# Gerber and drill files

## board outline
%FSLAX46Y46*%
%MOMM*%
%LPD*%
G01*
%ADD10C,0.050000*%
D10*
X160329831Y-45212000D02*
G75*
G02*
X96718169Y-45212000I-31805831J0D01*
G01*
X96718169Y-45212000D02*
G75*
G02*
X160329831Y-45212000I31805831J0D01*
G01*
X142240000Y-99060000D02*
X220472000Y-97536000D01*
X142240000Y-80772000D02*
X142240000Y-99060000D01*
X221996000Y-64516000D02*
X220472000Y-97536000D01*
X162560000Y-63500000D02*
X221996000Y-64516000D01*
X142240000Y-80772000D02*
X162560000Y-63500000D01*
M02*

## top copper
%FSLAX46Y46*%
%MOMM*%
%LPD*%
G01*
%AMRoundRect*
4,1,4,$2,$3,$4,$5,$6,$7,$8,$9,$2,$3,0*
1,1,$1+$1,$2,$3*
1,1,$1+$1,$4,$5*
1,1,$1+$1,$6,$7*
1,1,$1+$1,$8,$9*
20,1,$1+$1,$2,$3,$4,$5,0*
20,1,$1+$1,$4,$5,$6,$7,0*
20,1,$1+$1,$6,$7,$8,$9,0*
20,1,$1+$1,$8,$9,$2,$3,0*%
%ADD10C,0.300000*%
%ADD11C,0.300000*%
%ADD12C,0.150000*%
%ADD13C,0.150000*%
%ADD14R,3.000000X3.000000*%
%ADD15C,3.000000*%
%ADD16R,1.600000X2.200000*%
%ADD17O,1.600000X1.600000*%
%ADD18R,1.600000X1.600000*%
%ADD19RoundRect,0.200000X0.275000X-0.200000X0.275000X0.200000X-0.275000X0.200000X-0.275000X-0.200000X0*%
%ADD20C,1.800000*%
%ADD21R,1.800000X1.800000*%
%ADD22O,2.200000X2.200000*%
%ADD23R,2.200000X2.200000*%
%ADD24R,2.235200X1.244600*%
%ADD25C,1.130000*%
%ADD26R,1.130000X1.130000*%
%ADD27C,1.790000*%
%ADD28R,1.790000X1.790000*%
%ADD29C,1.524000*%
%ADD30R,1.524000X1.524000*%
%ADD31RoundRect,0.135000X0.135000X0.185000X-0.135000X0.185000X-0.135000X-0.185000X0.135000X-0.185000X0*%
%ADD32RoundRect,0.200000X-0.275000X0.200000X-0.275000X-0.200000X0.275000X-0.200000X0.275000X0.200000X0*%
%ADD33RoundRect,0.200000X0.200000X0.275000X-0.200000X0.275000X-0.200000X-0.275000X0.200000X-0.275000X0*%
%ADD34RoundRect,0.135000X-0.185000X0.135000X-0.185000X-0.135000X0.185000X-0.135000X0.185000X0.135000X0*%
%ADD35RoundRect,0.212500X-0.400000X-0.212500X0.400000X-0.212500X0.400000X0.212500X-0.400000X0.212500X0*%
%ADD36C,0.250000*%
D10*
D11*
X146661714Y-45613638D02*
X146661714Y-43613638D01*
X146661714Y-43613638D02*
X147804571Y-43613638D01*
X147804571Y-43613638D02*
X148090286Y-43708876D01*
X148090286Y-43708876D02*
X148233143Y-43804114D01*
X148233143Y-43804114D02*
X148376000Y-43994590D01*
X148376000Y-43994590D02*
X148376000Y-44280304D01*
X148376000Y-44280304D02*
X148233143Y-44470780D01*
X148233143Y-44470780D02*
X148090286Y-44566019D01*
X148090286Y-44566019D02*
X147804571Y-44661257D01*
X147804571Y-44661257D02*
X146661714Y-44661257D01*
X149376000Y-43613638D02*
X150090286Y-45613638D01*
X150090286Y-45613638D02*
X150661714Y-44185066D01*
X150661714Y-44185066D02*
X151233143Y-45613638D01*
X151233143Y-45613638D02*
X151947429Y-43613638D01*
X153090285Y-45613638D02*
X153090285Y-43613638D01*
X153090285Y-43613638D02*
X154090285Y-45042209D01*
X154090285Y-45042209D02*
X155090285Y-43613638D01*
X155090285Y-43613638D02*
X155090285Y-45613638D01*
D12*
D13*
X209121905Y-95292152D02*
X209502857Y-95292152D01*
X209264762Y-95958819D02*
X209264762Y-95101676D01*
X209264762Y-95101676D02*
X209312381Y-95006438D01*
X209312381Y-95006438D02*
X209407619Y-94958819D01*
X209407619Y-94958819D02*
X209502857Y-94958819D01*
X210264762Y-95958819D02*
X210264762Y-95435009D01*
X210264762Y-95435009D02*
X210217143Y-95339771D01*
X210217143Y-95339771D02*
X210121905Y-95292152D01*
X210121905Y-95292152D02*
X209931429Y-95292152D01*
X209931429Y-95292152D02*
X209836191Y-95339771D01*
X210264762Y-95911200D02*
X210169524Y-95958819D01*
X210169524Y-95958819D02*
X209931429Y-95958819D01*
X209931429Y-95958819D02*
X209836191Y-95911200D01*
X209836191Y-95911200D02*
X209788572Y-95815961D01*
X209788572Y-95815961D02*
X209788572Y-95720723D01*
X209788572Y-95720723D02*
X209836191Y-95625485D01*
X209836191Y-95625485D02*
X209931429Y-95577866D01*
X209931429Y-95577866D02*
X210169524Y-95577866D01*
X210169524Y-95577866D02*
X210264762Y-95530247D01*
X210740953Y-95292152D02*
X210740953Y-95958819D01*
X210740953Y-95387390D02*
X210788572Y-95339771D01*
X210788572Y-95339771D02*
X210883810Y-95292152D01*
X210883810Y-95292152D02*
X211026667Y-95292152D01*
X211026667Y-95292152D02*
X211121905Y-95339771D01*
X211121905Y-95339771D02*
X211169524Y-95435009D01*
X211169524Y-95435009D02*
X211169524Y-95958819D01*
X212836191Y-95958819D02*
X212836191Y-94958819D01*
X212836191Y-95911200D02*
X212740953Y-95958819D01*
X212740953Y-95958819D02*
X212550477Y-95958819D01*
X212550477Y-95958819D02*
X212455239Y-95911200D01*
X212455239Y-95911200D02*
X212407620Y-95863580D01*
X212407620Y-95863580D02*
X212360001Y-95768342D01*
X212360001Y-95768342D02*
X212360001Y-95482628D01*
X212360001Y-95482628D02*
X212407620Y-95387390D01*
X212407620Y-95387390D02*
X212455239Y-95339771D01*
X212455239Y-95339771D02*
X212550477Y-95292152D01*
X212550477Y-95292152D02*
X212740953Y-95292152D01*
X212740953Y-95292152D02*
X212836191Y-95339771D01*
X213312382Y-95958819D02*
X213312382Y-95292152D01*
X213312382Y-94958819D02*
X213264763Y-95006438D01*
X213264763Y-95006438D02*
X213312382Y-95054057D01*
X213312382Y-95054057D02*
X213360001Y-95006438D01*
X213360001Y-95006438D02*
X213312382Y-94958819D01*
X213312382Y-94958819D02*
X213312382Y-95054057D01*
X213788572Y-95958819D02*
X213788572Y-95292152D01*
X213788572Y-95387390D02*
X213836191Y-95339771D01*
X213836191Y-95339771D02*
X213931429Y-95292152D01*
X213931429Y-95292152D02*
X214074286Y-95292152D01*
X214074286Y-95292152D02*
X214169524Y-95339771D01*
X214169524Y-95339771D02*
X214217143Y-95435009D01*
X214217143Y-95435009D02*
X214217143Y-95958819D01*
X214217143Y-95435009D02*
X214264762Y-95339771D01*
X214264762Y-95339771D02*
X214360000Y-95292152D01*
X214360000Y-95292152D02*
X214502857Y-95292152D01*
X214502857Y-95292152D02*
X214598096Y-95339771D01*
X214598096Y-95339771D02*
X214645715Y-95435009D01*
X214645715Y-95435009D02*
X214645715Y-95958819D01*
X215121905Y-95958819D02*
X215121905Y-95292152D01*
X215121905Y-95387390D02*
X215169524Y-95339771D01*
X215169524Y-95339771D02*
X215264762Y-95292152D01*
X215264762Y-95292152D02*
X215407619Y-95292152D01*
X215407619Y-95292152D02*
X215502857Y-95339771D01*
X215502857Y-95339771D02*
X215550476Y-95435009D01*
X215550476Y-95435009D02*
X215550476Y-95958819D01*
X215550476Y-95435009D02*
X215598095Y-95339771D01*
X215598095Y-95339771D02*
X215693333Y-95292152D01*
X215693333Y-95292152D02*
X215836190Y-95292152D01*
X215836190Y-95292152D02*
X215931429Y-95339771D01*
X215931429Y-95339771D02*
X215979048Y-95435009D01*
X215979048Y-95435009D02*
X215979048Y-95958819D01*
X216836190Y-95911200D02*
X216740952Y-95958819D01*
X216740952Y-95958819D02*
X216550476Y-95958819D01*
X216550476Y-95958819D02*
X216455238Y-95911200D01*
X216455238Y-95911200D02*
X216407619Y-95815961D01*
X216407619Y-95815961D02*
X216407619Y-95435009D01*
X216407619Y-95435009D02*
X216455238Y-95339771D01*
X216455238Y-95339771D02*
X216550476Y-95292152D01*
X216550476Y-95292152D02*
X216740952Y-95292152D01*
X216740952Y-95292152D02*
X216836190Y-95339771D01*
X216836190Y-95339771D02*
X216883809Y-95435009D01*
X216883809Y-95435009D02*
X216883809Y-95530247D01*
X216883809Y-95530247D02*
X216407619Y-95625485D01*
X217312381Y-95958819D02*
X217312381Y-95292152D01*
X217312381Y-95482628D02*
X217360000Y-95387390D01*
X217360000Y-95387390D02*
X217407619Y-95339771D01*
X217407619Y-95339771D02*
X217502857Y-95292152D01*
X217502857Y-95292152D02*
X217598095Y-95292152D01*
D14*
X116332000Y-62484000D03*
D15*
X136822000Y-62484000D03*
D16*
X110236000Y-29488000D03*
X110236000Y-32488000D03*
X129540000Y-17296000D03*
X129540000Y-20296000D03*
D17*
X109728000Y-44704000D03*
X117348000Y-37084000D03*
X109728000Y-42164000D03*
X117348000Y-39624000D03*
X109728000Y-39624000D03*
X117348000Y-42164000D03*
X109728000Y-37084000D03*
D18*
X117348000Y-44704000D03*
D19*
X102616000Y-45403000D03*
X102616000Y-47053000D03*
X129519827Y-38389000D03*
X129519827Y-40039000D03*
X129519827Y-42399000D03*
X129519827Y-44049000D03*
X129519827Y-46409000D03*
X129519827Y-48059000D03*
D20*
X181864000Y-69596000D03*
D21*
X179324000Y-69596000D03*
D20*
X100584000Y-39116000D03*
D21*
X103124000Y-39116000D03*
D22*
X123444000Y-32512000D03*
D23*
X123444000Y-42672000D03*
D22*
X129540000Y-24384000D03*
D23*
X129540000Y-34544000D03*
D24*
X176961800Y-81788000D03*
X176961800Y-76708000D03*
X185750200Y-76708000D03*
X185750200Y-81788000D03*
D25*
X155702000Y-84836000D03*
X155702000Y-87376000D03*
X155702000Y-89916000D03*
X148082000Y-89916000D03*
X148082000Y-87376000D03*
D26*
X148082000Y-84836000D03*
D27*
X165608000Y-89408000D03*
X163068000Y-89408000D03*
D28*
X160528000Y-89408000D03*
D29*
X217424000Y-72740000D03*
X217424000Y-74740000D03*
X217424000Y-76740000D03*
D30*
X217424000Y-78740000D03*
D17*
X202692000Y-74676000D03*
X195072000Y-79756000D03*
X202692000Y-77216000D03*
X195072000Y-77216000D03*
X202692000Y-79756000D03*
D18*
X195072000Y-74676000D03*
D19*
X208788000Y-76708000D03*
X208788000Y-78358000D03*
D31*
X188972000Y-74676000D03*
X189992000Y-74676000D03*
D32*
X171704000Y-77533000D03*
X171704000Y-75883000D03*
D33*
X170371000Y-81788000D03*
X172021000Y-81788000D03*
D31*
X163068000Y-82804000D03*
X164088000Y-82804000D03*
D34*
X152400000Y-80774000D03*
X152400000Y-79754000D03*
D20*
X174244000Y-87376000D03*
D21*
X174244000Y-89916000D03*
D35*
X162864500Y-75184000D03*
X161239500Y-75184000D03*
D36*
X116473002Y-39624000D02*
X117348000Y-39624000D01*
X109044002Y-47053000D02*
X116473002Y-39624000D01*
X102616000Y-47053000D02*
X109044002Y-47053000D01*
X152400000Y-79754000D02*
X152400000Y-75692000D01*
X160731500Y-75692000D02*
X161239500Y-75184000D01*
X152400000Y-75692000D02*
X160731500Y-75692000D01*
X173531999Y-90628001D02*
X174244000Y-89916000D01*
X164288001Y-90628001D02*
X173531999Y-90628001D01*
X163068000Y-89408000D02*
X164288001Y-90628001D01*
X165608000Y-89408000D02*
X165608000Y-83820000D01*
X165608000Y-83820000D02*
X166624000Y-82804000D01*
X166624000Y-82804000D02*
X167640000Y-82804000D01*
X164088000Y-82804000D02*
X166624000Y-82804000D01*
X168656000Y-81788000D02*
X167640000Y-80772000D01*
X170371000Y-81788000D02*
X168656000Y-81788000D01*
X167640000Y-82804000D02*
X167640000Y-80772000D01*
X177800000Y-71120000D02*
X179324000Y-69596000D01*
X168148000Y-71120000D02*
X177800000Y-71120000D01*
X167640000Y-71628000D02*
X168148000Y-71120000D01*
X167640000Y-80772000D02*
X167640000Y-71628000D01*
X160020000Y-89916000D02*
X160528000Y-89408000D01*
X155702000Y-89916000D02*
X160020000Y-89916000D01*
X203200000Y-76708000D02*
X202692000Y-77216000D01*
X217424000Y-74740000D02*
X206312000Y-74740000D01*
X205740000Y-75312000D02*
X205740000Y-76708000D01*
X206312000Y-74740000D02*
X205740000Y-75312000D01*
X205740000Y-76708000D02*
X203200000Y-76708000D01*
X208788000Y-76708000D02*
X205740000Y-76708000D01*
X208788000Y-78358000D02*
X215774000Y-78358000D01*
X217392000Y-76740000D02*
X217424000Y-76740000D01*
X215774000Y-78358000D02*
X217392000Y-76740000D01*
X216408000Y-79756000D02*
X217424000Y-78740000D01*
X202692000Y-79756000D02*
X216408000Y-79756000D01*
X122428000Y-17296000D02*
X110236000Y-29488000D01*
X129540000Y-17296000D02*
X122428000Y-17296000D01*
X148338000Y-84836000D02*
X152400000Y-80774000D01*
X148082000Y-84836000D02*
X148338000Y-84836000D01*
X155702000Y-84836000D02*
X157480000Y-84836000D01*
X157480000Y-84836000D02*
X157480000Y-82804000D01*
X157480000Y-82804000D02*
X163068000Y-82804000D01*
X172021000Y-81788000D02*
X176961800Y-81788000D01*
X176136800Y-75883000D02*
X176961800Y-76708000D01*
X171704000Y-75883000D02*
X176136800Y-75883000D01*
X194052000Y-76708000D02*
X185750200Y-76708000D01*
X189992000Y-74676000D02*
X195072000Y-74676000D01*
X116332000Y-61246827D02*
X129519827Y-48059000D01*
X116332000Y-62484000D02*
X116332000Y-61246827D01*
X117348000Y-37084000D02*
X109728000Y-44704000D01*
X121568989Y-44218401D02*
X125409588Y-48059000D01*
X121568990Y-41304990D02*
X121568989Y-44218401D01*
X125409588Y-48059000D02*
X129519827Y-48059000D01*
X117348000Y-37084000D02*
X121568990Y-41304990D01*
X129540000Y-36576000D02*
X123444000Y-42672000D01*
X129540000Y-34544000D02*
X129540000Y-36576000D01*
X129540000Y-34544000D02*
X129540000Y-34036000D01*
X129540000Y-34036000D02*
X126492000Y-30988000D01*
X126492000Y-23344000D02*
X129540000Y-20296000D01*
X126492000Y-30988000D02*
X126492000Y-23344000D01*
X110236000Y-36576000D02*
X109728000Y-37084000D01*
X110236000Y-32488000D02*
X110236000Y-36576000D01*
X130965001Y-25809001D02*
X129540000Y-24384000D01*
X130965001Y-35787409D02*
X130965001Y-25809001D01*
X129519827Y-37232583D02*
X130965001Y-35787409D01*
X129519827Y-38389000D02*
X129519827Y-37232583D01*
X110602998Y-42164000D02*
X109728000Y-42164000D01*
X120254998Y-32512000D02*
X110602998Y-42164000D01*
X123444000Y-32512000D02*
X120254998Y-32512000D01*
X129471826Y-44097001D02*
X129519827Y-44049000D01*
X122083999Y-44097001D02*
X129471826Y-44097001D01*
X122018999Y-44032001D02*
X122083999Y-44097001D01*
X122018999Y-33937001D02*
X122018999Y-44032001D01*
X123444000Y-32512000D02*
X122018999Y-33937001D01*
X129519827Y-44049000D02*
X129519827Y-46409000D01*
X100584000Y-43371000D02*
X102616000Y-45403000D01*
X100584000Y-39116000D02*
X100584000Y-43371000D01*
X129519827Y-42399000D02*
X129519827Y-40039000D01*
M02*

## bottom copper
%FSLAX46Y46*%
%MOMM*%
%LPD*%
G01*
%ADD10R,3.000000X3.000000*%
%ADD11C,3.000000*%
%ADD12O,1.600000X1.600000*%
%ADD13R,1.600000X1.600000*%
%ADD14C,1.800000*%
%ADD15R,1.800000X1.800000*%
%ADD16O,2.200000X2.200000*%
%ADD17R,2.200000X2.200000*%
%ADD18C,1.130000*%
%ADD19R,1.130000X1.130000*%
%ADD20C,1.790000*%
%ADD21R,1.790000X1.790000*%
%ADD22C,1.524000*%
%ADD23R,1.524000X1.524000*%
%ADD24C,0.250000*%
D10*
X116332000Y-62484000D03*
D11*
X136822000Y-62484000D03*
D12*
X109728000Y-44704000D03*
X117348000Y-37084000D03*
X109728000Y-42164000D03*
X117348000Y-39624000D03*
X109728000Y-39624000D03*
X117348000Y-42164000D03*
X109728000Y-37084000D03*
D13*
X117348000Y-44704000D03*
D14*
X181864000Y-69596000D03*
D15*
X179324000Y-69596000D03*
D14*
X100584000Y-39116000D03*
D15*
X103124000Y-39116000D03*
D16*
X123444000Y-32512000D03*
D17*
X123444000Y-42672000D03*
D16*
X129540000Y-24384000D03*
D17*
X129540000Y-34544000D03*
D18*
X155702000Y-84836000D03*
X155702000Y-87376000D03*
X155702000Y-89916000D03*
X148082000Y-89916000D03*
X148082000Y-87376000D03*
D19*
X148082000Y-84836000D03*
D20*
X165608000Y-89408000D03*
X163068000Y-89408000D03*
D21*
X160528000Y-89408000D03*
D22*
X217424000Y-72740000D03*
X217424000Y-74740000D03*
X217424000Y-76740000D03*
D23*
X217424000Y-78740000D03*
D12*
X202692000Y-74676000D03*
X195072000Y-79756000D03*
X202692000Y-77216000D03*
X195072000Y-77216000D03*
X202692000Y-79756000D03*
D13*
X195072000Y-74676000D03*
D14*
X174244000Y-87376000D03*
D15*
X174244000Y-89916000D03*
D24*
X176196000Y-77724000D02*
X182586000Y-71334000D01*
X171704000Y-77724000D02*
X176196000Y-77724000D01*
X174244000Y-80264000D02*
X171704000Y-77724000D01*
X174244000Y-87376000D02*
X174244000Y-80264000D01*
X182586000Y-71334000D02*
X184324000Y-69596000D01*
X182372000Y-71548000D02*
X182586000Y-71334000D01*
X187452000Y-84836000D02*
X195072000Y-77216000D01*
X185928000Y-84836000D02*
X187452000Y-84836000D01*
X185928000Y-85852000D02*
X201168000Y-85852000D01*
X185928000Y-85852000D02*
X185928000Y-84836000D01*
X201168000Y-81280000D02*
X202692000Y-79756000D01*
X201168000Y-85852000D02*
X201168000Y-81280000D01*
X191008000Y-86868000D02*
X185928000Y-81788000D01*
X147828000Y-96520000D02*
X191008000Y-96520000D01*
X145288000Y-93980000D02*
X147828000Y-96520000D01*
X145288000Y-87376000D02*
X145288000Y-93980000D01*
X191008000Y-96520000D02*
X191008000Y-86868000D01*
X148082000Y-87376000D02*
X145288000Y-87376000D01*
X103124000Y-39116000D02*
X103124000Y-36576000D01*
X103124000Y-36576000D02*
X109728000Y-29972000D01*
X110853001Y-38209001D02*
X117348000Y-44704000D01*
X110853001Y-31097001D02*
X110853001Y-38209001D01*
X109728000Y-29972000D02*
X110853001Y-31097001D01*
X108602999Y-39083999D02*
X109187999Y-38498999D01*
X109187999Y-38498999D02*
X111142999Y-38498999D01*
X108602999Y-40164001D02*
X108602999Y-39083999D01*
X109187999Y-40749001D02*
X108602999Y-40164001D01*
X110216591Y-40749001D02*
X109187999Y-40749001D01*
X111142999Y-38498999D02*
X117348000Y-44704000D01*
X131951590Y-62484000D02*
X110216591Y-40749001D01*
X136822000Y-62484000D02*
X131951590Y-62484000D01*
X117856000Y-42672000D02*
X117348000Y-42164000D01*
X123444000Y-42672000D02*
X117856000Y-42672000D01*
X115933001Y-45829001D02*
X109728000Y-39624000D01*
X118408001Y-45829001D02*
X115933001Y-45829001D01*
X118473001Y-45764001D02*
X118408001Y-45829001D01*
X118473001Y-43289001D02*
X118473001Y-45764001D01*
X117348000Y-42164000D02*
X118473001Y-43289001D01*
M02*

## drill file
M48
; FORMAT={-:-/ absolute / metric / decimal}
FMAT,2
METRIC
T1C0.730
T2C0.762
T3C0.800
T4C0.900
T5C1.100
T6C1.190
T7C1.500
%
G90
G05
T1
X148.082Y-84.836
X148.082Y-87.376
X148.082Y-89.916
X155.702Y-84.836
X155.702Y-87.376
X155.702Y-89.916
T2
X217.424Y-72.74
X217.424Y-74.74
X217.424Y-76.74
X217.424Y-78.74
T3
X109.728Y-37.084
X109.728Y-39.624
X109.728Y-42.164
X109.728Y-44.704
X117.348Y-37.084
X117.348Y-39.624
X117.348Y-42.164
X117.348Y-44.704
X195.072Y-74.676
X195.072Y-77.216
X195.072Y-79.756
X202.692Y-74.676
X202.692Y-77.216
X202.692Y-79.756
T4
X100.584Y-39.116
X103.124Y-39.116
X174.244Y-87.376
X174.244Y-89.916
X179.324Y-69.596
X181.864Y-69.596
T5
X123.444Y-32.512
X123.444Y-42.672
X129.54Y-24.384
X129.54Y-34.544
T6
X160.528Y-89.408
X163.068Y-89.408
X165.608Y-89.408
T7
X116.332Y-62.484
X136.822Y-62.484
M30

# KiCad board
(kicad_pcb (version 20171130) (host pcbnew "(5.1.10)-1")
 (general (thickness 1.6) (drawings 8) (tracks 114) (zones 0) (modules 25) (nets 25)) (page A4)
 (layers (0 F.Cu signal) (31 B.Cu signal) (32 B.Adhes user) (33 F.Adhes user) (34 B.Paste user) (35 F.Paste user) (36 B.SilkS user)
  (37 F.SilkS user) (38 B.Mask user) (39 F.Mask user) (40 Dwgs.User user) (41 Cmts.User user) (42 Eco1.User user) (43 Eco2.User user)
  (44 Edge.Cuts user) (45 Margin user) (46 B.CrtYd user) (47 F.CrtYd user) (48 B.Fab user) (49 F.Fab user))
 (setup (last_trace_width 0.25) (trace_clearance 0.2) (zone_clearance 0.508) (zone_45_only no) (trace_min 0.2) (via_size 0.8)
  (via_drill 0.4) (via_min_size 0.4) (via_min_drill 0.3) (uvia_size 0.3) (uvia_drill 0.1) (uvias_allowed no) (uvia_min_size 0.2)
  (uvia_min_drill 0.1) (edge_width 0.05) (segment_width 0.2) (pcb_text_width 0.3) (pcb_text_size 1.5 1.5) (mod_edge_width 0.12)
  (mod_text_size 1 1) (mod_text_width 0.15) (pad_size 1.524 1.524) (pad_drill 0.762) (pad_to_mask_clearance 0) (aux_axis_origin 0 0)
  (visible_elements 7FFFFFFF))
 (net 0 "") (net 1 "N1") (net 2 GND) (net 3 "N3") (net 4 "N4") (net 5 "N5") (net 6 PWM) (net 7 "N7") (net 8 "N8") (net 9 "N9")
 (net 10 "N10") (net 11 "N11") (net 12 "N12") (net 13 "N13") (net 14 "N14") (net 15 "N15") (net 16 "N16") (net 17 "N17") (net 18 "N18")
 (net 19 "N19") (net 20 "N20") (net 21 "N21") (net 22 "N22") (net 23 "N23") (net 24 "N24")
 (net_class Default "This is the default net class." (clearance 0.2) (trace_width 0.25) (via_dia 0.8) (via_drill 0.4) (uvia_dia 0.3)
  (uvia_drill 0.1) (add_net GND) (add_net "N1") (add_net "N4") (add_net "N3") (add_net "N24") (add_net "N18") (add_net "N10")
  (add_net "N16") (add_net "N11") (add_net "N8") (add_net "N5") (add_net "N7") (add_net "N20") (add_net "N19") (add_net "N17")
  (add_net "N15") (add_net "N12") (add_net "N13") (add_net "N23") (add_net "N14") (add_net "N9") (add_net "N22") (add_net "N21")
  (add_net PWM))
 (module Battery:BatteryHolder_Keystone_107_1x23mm (layer F.Cu) (at 116.332 62.484)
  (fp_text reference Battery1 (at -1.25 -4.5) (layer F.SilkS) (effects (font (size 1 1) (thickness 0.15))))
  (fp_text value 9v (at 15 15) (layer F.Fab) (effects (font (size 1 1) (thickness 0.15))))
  (pad 1 thru_hole rect (at 0 0) (size 3 3) (drill 1.5) (layers *.Cu *.Mask) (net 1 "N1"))
  (pad 2 thru_hole circle (at 20.49 0) (size 3 3) (drill 1.5) (layers *.Cu *.Mask) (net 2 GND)))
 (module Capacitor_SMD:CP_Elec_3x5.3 (layer F.Cu) (at 110.236 30.988 90)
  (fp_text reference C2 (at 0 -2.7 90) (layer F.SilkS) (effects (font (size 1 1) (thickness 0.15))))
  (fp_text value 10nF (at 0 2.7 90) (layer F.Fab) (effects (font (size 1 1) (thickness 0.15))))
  (pad 2 smd rect (at 1.5 0 90) (size 2.2 1.6) (layers F.Cu F.Paste F.Mask) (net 2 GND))
  (pad 1 smd rect (at -1.5 0 90) (size 2.2 1.6) (layers F.Cu F.Paste F.Mask) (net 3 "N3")))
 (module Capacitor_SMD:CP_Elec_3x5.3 (layer F.Cu) (at 129.54 18.796 90)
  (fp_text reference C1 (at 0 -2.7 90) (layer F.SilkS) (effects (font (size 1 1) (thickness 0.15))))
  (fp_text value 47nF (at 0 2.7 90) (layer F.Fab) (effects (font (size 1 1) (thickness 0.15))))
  (pad 2 smd rect (at 1.5 0 90) (size 2.2 1.6) (layers F.Cu F.Paste F.Mask) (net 2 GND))
  (pad 1 smd rect (at -1.5 0 90) (size 2.2 1.6) (layers F.Cu F.Paste F.Mask) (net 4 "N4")))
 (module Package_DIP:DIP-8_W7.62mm (layer F.Cu) (at 117.348 44.704 180)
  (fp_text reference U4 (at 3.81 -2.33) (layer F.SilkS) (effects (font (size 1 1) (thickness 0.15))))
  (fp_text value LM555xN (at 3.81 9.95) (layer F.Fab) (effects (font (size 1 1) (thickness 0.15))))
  (pad 8 thru_hole oval (at 7.62 0 180) (size 1.6 1.6) (drill 0.8) (layers *.Cu *.Mask) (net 1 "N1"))
  (pad 4 thru_hole oval (at 0 7.62 180) (size 1.6 1.6) (drill 0.8) (layers *.Cu *.Mask) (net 1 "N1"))
  (pad 7 thru_hole oval (at 7.62 2.54 180) (size 1.6 1.6) (drill 0.8) (layers *.Cu *.Mask) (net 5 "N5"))
  (pad 3 thru_hole oval (at 0 5.08 180) (size 1.6 1.6) (drill 0.8) (layers *.Cu *.Mask) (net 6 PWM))
  (pad 6 thru_hole oval (at 7.62 5.08 180) (size 1.6 1.6) (drill 0.8) (layers *.Cu *.Mask) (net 4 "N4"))
  (pad 2 thru_hole oval (at 0 2.54 180) (size 1.6 1.6) (drill 0.8) (layers *.Cu *.Mask) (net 4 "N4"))
  (pad 5 thru_hole oval (at 7.62 7.62 180) (size 1.6 1.6) (drill 0.8) (layers *.Cu *.Mask) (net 3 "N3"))
  (pad 1 thru_hole rect (at 0 0 180) (size 1.6 1.6) (drill 0.8) (layers *.Cu *.Mask) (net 2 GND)))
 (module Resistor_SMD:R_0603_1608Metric (layer F.Cu) (at 102.616 46.228 90)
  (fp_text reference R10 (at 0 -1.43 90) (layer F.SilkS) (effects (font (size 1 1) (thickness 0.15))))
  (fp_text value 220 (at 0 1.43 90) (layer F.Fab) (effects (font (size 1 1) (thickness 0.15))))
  (pad 2 smd roundrect (at 0.825 0 90) (size 0.8 0.95) (layers F.Cu F.Paste F.Mask) (roundrect_rratio 0.25) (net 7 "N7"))
  (pad 1 smd roundrect (at -0.825 0 90) (size 0.8 0.95) (layers F.Cu F.Paste F.Mask) (roundrect_rratio 0.25) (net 6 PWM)))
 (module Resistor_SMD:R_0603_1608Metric (layer F.Cu) (at 129.519827 39.214 90)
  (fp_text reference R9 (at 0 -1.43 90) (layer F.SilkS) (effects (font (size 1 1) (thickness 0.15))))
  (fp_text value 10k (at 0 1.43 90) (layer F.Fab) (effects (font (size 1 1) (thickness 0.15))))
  (pad 2 smd roundrect (at 0.825 0 90) (size 0.8 0.95) (layers F.Cu F.Paste F.Mask) (roundrect_rratio 0.25) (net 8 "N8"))
  (pad 1 smd roundrect (at -0.825 0 90) (size 0.8 0.95) (layers F.Cu F.Paste F.Mask) (roundrect_rratio 0.25) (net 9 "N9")))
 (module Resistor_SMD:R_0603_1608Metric (layer F.Cu) (at 129.519827 43.224 90)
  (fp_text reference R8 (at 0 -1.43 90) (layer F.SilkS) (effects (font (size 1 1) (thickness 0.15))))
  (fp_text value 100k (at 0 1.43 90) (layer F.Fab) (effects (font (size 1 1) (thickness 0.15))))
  (pad 2 smd roundrect (at 0.825 0 90) (size 0.8 0.95) (layers F.Cu F.Paste F.Mask) (roundrect_rratio 0.25) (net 9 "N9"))
  (pad 1 smd roundrect (at -0.825 0 90) (size 0.8 0.95) (layers F.Cu F.Paste F.Mask) (roundrect_rratio 0.25) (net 5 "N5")))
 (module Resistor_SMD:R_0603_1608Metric (layer F.Cu) (at 129.519827 47.234 90)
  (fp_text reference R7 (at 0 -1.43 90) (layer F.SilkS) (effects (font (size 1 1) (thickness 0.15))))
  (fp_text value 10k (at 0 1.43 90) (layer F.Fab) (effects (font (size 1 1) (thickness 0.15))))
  (pad 2 smd roundrect (at 0.825 0 90) (size 0.8 0.95) (layers F.Cu F.Paste F.Mask) (roundrect_rratio 0.25) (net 5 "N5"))
  (pad 1 smd roundrect (at -0.825 0 90) (size 0.8 0.95) (layers F.Cu F.Paste F.Mask) (roundrect_rratio 0.25) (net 1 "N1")))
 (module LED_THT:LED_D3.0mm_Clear (layer F.Cu) (at 179.324 69.596)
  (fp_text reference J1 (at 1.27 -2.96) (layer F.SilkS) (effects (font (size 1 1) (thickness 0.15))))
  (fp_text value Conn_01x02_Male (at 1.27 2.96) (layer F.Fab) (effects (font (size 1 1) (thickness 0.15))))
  (pad 2 thru_hole circle (at 2.54 0) (size 1.8 1.8) (drill 0.9) (layers *.Cu *.Mask) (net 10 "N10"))
  (pad 1 thru_hole rect (at 0 0) (size 1.8 1.8) (drill 0.9) (layers *.Cu *.Mask) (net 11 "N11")))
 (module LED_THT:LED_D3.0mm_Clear (layer F.Cu) (at 103.124 39.116 180)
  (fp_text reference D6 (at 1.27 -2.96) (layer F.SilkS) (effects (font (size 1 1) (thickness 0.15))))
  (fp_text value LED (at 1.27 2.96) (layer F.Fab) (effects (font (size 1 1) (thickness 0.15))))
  (pad 2 thru_hole circle (at 2.54 0 180) (size 1.8 1.8) (drill 0.9) (layers *.Cu *.Mask) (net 7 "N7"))
  (pad 1 thru_hole rect (at 0 0 180) (size 1.8 1.8) (drill 0.9) (layers *.Cu *.Mask) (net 2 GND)))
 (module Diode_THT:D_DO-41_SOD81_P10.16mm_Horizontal (layer F.Cu) (at 123.444 42.672 90)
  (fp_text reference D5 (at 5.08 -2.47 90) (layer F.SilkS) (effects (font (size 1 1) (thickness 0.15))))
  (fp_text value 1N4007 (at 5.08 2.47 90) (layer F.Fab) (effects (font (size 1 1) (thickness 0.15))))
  (pad 2 thru_hole oval (at 10.16 0 90) (size 2.2 2.2) (drill 1.1) (layers *.Cu *.Mask) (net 5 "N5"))
  (pad 1 thru_hole rect (at 0 0 90) (size 2.2 2.2) (drill 1.1) (layers *.Cu *.Mask) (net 4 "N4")))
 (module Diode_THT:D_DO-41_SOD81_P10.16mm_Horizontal (layer F.Cu) (at 129.54 34.544 90)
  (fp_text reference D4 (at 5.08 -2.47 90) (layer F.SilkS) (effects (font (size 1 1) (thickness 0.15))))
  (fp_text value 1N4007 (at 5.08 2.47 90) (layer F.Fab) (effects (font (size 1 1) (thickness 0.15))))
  (pad 2 thru_hole oval (at 10.16 0 90) (size 2.2 2.2) (drill 1.1) (layers *.Cu *.Mask) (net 8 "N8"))
  (pad 1 thru_hole rect (at 0 0 90) (size 2.2 2.2) (drill 1.1) (layers *.Cu *.Mask) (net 4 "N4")))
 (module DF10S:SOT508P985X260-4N (layer F.Cu) (at 181.356 79.248 180)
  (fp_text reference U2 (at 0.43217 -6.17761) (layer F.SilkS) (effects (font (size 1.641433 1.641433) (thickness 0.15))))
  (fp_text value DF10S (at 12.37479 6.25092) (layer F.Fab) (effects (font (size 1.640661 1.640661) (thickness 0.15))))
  (pad 4 smd rect (at 4.3942 -2.54 180) (size 2.2352 1.2446) (layers F.Cu F.Paste F.Mask) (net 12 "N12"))
  (pad 3 smd rect (at 4.3942 2.54 180) (size 2.2352 1.2446) (layers F.Cu F.Paste F.Mask) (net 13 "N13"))
  (pad 2 smd rect (at -4.3942 2.54 180) (size 2.2352 1.2446) (layers F.Cu F.Paste F.Mask) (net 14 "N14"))
  (pad 1 smd rect (at -4.3942 -2.54 180) (size 2.2352 1.2446) (layers F.Cu F.Paste F.Mask) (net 2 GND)))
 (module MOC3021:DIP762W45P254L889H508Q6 (layer F.Cu) (at 151.892 87.376)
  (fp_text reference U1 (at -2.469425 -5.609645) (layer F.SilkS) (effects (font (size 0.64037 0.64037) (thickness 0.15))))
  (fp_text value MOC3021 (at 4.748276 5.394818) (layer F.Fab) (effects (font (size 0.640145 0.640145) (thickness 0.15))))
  (pad 6 thru_hole circle (at 3.81 -2.54) (size 1.13 1.13) (drill 0.73) (layers *.Cu *.Mask) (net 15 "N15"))
  (pad 5 thru_hole circle (at 3.81 0) (size 1.13 1.13) (drill 0.73) (layers *.Cu *.Mask))
  (pad 4 thru_hole circle (at 3.81 2.54) (size 1.13 1.13) (drill 0.73) (layers *.Cu *.Mask) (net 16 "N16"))
  (pad 3 thru_hole circle (at -3.81 2.54) (size 1.13 1.13) (drill 0.73) (layers *.Cu *.Mask))
  (pad 2 thru_hole circle (at -3.81 0) (size 1.13 1.13) (drill 0.73) (layers *.Cu *.Mask) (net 2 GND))
  (pad 1 thru_hole rect (at -3.81 -2.54) (size 1.13 1.13) (drill 0.73) (layers *.Cu *.Mask) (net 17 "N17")))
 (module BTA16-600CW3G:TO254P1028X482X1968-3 (layer F.Cu) (at 160.528 89.408)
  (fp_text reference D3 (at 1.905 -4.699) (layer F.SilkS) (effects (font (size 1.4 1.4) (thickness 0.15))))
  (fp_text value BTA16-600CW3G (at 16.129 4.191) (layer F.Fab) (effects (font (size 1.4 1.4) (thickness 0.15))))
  (pad 3 thru_hole circle (at 5.08 0) (size 1.79 1.79) (drill 1.19) (layers *.Cu *.Mask) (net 11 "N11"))
  (pad 2 thru_hole circle (at 2.54 0) (size 1.79 1.79) (drill 1.19) (layers *.Cu *.Mask) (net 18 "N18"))
  (pad 1 thru_hole rect (at 0 0) (size 1.79 1.79) (drill 1.19) (layers *.Cu *.Mask) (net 16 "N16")))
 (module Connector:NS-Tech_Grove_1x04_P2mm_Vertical (layer F.Cu) (at 217.424 78.74 180)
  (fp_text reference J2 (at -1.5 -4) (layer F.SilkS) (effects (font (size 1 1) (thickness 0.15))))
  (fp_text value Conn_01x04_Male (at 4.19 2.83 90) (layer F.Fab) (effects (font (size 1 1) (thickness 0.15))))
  (pad 4 thru_hole circle (at 0 6 180) (size 1.524 1.524) (drill 0.762) (layers *.Cu *.Mask) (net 6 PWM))
  (pad 3 thru_hole circle (at 0 4 180) (size 1.524 1.524) (drill 0.762) (layers *.Cu *.Mask) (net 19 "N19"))
  (pad 2 thru_hole circle (at 0 2 180) (size 1.524 1.524) (drill 0.762) (layers *.Cu *.Mask) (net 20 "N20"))
  (pad 1 thru_hole rect (at 0 0 180) (size 1.524 1.524) (drill 0.762) (layers *.Cu *.Mask) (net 2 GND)))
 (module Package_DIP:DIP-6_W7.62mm (layer F.Cu) (at 195.072 74.676)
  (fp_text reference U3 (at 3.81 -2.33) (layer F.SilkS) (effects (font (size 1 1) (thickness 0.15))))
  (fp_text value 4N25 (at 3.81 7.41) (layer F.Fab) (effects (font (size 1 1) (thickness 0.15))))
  (pad 6 thru_hole oval (at 7.62 0) (size 1.6 1.6) (drill 0.8) (layers *.Cu *.Mask) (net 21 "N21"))
  (pad 3 thru_hole oval (at 0 5.08) (size 1.6 1.6) (drill 0.8) (layers *.Cu *.Mask) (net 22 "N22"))
  (pad 5 thru_hole oval (at 7.62 2.54) (size 1.6 1.6) (drill 0.8) (layers *.Cu *.Mask) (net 19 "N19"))
  (pad 2 thru_hole oval (at 0 2.54) (size 1.6 1.6) (drill 0.8) (layers *.Cu *.Mask) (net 2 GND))
  (pad 4 thru_hole oval (at 7.62 5.08) (size 1.6 1.6) (drill 0.8) (layers *.Cu *.Mask) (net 2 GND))
  (pad 1 thru_hole rect (at 0 0) (size 1.6 1.6) (drill 0.8) (layers *.Cu *.Mask) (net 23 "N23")))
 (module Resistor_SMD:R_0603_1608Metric (layer F.Cu) (at 208.788 77.533 90)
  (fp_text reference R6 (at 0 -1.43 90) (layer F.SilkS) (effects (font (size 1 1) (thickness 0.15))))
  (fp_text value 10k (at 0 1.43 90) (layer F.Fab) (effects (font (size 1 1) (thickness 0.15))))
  (pad 2 smd roundrect (at 0.825 0 90) (size 0.8 0.95) (layers F.Cu F.Paste F.Mask) (roundrect_rratio 0.25) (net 19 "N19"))
  (pad 1 smd roundrect (at -0.825 0 90) (size 0.8 0.95) (layers F.Cu F.Paste F.Mask) (roundrect_rratio 0.25) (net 20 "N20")))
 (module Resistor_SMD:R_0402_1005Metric (layer F.Cu) (at 189.482 74.676 180)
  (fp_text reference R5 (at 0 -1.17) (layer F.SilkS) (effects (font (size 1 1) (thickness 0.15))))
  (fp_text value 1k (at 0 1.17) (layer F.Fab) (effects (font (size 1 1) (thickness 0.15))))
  (pad 2 smd roundrect (at 0.51 0 180) (size 0.54 0.64) (layers F.Cu F.Paste F.Mask) (roundrect_rratio 0.25) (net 14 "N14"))
  (pad 1 smd roundrect (at -0.51 0 180) (size 0.54 0.64) (layers F.Cu F.Paste F.Mask) (roundrect_rratio 0.25) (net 23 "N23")))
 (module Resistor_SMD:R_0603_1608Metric (layer F.Cu) (at 171.704 76.708 270)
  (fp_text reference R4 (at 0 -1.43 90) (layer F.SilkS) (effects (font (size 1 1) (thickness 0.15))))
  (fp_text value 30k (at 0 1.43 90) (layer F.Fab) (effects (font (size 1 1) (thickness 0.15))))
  (pad 2 smd roundrect (at 0.825 0 270) (size 0.8 0.95) (layers F.Cu F.Paste F.Mask) (roundrect_rratio 0.25) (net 10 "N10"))
  (pad 1 smd roundrect (at -0.825 0 270) (size 0.8 0.95) (layers F.Cu F.Paste F.Mask) (roundrect_rratio 0.25) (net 13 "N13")))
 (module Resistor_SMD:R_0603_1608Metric (layer F.Cu) (at 171.196 81.788 180)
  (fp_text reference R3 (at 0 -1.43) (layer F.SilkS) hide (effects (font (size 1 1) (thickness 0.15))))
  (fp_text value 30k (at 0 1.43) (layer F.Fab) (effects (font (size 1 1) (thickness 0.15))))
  (pad 2 smd roundrect (at 0.825 0 180) (size 0.8 0.95) (layers F.Cu F.Paste F.Mask) (roundrect_rratio 0.25) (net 11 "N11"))
  (pad 1 smd roundrect (at -0.825 0 180) (size 0.8 0.95) (layers F.Cu F.Paste F.Mask) (roundrect_rratio 0.25) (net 12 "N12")))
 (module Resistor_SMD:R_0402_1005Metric (layer F.Cu) (at 163.578 82.804 180)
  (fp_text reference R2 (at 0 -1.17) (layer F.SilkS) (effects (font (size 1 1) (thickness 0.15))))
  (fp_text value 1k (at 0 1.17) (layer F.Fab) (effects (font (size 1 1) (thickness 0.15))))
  (pad 2 smd roundrect (at 0.51 0 180) (size 0.54 0.64) (layers F.Cu F.Paste F.Mask) (roundrect_rratio 0.25) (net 15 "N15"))
  (pad 1 smd roundrect (at -0.51 0 180) (size 0.54 0.64) (layers F.Cu F.Paste F.Mask) (roundrect_rratio 0.25) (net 11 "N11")))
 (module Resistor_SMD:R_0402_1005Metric (layer F.Cu) (at 152.4 80.264 270)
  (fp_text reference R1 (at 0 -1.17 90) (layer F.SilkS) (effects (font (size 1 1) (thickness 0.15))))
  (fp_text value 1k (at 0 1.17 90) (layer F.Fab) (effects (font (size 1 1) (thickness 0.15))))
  (pad 2 smd roundrect (at 0.51 0 270) (size 0.54 0.64) (layers F.Cu F.Paste F.Mask) (roundrect_rratio 0.25) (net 17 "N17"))
  (pad 1 smd roundrect (at -0.51 0 270) (size 0.54 0.64) (layers F.Cu F.Paste F.Mask) (roundrect_rratio 0.25) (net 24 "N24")))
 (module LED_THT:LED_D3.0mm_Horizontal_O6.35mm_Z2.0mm (layer F.Cu) (at 174.244 89.916 90)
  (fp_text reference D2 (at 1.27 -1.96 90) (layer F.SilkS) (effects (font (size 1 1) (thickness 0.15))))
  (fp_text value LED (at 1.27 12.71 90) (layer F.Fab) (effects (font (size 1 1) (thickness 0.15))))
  (pad 2 thru_hole circle (at 2.54 0 90) (size 1.8 1.8) (drill 0.9) (layers *.Cu *.Mask) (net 10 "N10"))
  (pad 1 thru_hole rect (at 0 0 90) (size 1.8 1.8) (drill 0.9) (layers *.Cu *.Mask) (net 18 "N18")))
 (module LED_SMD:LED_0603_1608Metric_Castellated (layer F.Cu) (at 162.052 75.184)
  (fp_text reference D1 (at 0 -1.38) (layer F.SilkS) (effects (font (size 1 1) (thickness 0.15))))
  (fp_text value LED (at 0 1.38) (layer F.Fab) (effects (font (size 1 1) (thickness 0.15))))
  (pad 2 smd roundrect (at 0.8125 0) (size 1.225 0.85) (layers F.Cu F.Paste F.Mask) (roundrect_rratio 0.25) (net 6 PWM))
  (pad 1 smd roundrect (at -0.8125 0) (size 1.225 0.85) (layers F.Cu F.Paste F.Mask) (roundrect_rratio 0.25) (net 24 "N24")))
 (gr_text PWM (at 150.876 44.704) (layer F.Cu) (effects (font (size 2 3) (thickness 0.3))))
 (gr_circle (center 128.524 45.212) (end 114.3 16.764) (layer Edge.Cuts) (width 0.05))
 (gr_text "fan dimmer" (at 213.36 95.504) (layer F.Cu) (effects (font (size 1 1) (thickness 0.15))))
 (gr_line (start 142.24 99.06) (end 220.472 97.536) (layer Edge.Cuts) (width 0.05))
 (gr_line (start 142.24 80.772) (end 142.24 99.06) (layer Edge.Cuts) (width 0.05))
 (gr_line (start 221.996 64.516) (end 220.472 97.536) (layer Edge.Cuts) (width 0.05))
 (gr_line (start 162.56 63.5) (end 221.996 64.516) (layer Edge.Cuts) (width 0.05))
 (gr_line (start 142.24 80.772) (end 162.56 63.5) (layer Edge.Cuts) (width 0.05))
 (segment (start 116.473002 39.624) (end 117.348 39.624) (width 0.25) (layer F.Cu) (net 6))
 (segment (start 109.044002 47.053) (end 116.473002 39.624) (width 0.25) (layer F.Cu) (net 6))
 (segment (start 102.616 47.053) (end 109.044002 47.053) (width 0.25) (layer F.Cu) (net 6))
 (segment (start 152.4 79.754) (end 152.4 75.692) (width 0.25) (layer F.Cu) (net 24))
 (segment (start 160.7315 75.692) (end 161.2395 75.184) (width 0.25) (layer F.Cu) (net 24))
 (segment (start 152.4 75.692) (end 160.7315 75.692) (width 0.25) (layer F.Cu) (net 24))
 (segment (start 176.196 77.724) (end 182.586 71.334) (width 0.25) (layer B.Cu) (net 10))
 (segment (start 171.704 77.724) (end 176.196 77.724) (width 0.25) (layer B.Cu) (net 10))
 (segment (start 174.244 80.264) (end 171.704 77.724) (width 0.25) (layer B.Cu) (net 10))
 (segment (start 174.244 87.376) (end 174.244 80.264) (width 0.25) (layer B.Cu) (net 10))
 (segment (start 182.586 71.334) (end 184.324 69.596) (width 0.25) (layer B.Cu) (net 10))
 (segment (start 182.372 71.548) (end 182.586 71.334) (width 0.25) (layer B.Cu) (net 10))
 (segment (start 173.531999 90.628001) (end 174.244 89.916) (width 0.25) (layer F.Cu) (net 18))
 (segment (start 164.288001 90.628001) (end 173.531999 90.628001) (width 0.25) (layer F.Cu) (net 18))
 (segment (start 163.068 89.408) (end 164.288001 90.628001) (width 0.25) (layer F.Cu) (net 18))
 (segment (start 165.608 89.408) (end 165.608 83.82) (width 0.25) (layer F.Cu) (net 11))
 (segment (start 165.608 83.82) (end 166.624 82.804) (width 0.25) (layer F.Cu) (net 11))
 (segment (start 166.624 82.804) (end 167.64 82.804) (width 0.25) (layer F.Cu) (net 11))
 (segment (start 164.088 82.804) (end 166.624 82.804) (width 0.25) (layer F.Cu) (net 11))
 (segment (start 168.656 81.788) (end 167.64 80.772) (width 0.25) (layer F.Cu) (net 11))
 (segment (start 170.371 81.788) (end 168.656 81.788) (width 0.25) (layer F.Cu) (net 11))
 (segment (start 167.64 82.804) (end 167.64 80.772) (width 0.25) (layer F.Cu) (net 11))
 (segment (start 177.8 71.12) (end 179.324 69.596) (width 0.25) (layer F.Cu) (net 11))
 (segment (start 168.148 71.12) (end 177.8 71.12) (width 0.25) (layer F.Cu) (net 11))
 (segment (start 167.64 71.628) (end 168.148 71.12) (width 0.25) (layer F.Cu) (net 11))
 (segment (start 167.64 80.772) (end 167.64 71.628) (width 0.25) (layer F.Cu) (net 11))
 (segment (start 160.02 89.916) (end 160.528 89.408) (width 0.25) (layer F.Cu) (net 16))
 (segment (start 155.702 89.916) (end 160.02 89.916) (width 0.25) (layer F.Cu) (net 16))
 (segment (start 203.2 76.708) (end 202.692 77.216) (width 0.25) (layer F.Cu) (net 19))
 (segment (start 217.424 74.74) (end 206.312 74.74) (width 0.25) (layer F.Cu) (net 19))
 (segment (start 205.74 75.312) (end 205.74 76.708) (width 0.25) (layer F.Cu) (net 19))
 (segment (start 206.312 74.74) (end 205.74 75.312) (width 0.25) (layer F.Cu) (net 19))
 (segment (start 205.74 76.708) (end 203.2 76.708) (width 0.25) (layer F.Cu) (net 19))
 (segment (start 208.788 76.708) (end 205.74 76.708) (width 0.25) (layer F.Cu) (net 19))
 (segment (start 208.788 78.358) (end 215.774 78.358) (width 0.25) (layer F.Cu) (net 20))
 (segment (start 217.392 76.74) (end 217.424 76.74) (width 0.25) (layer F.Cu) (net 20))
 (segment (start 215.774 78.358) (end 217.392 76.74) (width 0.25) (layer F.Cu) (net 20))
 (segment (start 216.408 79.756) (end 217.424 78.74) (width 0.25) (layer F.Cu) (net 2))
 (segment (start 202.692 79.756) (end 216.408 79.756) (width 0.25) (layer F.Cu) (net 2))
 (segment (start 187.452 84.836) (end 195.072 77.216) (width 0.25) (layer B.Cu) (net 2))
 (segment (start 185.928 84.836) (end 187.452 84.836) (width 0.25) (layer B.Cu) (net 2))
 (segment (start 185.928 85.852) (end 201.168 85.852) (width 0.25) (layer B.Cu) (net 2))
 (segment (start 185.928 85.852) (end 185.928 84.836) (width 0.25) (layer B.Cu) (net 2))
 (segment (start 201.168 81.28) (end 202.692 79.756) (width 0.25) (layer B.Cu) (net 2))
 (segment (start 201.168 85.852) (end 201.168 81.28) (width 0.25) (layer B.Cu) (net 2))
 (segment (start 191.008 86.868) (end 185.928 81.788) (width 0.25) (layer B.Cu) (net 2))
 (segment (start 147.828 96.52) (end 191.008 96.52) (width 0.25) (layer B.Cu) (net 2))
 (segment (start 145.288 93.98) (end 147.828 96.52) (width 0.25) (layer B.Cu) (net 2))
 (segment (start 145.288 87.376) (end 145.288 93.98) (width 0.25) (layer B.Cu) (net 2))
 (segment (start 191.008 96.52) (end 191.008 86.868) (width 0.25) (layer B.Cu) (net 2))
 (segment (start 148.082 87.376) (end 145.288 87.376) (width 0.25) (layer B.Cu) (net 2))
 (segment (start 103.124 39.116) (end 103.124 36.576) (width 0.25) (layer B.Cu) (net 2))
 (segment (start 103.124 36.576) (end 109.728 29.972) (width 0.25) (layer B.Cu) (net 2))
 (segment (start 110.853001 38.209001) (end 117.348 44.704) (width 0.25) (layer B.Cu) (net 2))
 (segment (start 110.853001 31.097001) (end 110.853001 38.209001) (width 0.25) (layer B.Cu) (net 2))
 (segment (start 109.728 29.972) (end 110.853001 31.097001) (width 0.25) (layer B.Cu) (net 2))
 (segment (start 122.428 17.296) (end 110.236 29.488) (width 0.25) (layer F.Cu) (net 2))
 (segment (start 129.54 17.296) (end 122.428 17.296) (width 0.25) (layer F.Cu) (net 2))
 (segment (start 108.602999 39.083999) (end 109.187999 38.498999) (width 0.25) (layer B.Cu) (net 2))
 (segment (start 109.187999 38.498999) (end 111.142999 38.498999) (width 0.25) (layer B.Cu) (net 2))
 (segment (start 108.602999 40.164001) (end 108.602999 39.083999) (width 0.25) (layer B.Cu) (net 2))
 (segment (start 109.187999 40.749001) (end 108.602999 40.164001) (width 0.25) (layer B.Cu) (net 2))
 (segment (start 110.216591 40.749001) (end 109.187999 40.749001) (width 0.25) (layer B.Cu) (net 2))
 (segment (start 111.142999 38.498999) (end 117.348 44.704) (width 0.25) (layer B.Cu) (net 2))
 (segment (start 131.95159 62.484) (end 110.216591 40.749001) (width 0.25) (layer B.Cu) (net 2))
 (segment (start 136.822 62.484) (end 131.95159 62.484) (width 0.25) (layer B.Cu) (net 2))
 (segment (start 148.338 84.836) (end 152.4 80.774) (width 0.25) (layer F.Cu) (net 17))
 (segment (start 148.082 84.836) (end 148.338 84.836) (width 0.25) (layer F.Cu) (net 17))
 (segment (start 155.702 84.836) (end 157.48 84.836) (width 0.25) (layer F.Cu) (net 15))
 (segment (start 157.48 84.836) (end 157.48 82.804) (width 0.25) (layer F.Cu) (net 15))
 (segment (start 157.48 82.804) (end 163.068 82.804) (width 0.25) (layer F.Cu) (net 15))
 (segment (start 172.021 81.788) (end 176.9618 81.788) (width 0.25) (layer F.Cu) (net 12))
 (segment (start 176.1368 75.883) (end 176.9618 76.708) (width 0.25) (layer F.Cu) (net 13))
 (segment (start 171.704 75.883) (end 176.1368 75.883) (width 0.25) (layer F.Cu) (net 13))
 (segment (start 194.052 76.708) (end 185.7502 76.708) (width 0.25) (layer F.Cu) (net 14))
 (segment (start 189.992 74.676) (end 195.072 74.676) (width 0.25) (layer F.Cu) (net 23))
 (segment (start 116.332 61.246827) (end 129.519827 48.059) (width 0.25) (layer F.Cu) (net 1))
 (segment (start 116.332 62.484) (end 116.332 61.246827) (width 0.25) (layer F.Cu) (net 1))
 (segment (start 117.348 37.084) (end 109.728 44.704) (width 0.25) (layer F.Cu) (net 1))
 (segment (start 121.568989 44.218401) (end 125.409588 48.059) (width 0.25) (layer F.Cu) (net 1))
 (segment (start 121.56899 41.30499) (end 121.568989 44.218401) (width 0.25) (layer F.Cu) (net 1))
 (segment (start 125.409588 48.059) (end 129.519827 48.059) (width 0.25) (layer F.Cu) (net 1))
 (segment (start 117.348 37.084) (end 121.56899 41.30499) (width 0.25) (layer F.Cu) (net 1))
 (segment (start 117.856 42.672) (end 117.348 42.164) (width 0.25) (layer B.Cu) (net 4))
 (segment (start 123.444 42.672) (end 117.856 42.672) (width 0.25) (layer B.Cu) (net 4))
 (segment (start 115.933001 45.829001) (end 109.728 39.624) (width 0.25) (layer B.Cu) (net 4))
 (segment (start 118.408001 45.829001) (end 115.933001 45.829001) (width 0.25) (layer B.Cu) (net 4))
 (segment (start 118.473001 45.764001) (end 118.408001 45.829001) (width 0.25) (layer B.Cu) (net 4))
 (segment (start 118.473001 43.289001) (end 118.473001 45.764001) (width 0.25) (layer B.Cu) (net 4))
 (segment (start 117.348 42.164) (end 118.473001 43.289001) (width 0.25) (layer B.Cu) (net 4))
 (segment (start 129.54 36.576) (end 123.444 42.672) (width 0.25) (layer F.Cu) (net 4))
 (segment (start 129.54 34.544) (end 129.54 36.576) (width 0.25) (layer F.Cu) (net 4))
 (segment (start 129.54 34.544) (end 129.54 34.036) (width 0.25) (layer F.Cu) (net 4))
 (segment (start 129.54 34.036) (end 126.492 30.988) (width 0.25) (layer F.Cu) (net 4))
 (segment (start 126.492 23.344) (end 129.54 20.296) (width 0.25) (layer F.Cu) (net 4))
 (segment (start 126.492 30.988) (end 126.492 23.344) (width 0.25) (layer F.Cu) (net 4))
 (segment (start 110.236 36.576) (end 109.728 37.084) (width 0.25) (layer F.Cu) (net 3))
 (segment (start 110.236 32.488) (end 110.236 36.576) (width 0.25) (layer F.Cu) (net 3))
 (segment (start 130.965001 25.809001) (end 129.54 24.384) (width 0.25) (layer F.Cu) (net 8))
 (segment (start 130.965001 35.787409) (end 130.965001 25.809001) (width 0.25) (layer F.Cu) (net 8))
 (segment (start 129.519827 37.232583) (end 130.965001 35.787409) (width 0.25) (layer F.Cu) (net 8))
 (segment (start 129.519827 38.389) (end 129.519827 37.232583) (width 0.25) (layer F.Cu) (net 8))
 (segment (start 110.602998 42.164) (end 109.728 42.164) (width 0.25) (layer F.Cu) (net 5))
 (segment (start 120.254998 32.512) (end 110.602998 42.164) (width 0.25) (layer F.Cu) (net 5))
 (segment (start 123.444 32.512) (end 120.254998 32.512) (width 0.25) (layer F.Cu) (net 5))
 (segment (start 129.471826 44.097001) (end 129.519827 44.049) (width 0.25) (layer F.Cu) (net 5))
 (segment (start 122.083999 44.097001) (end 129.471826 44.097001) (width 0.25) (layer F.Cu) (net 5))
 (segment (start 122.018999 44.032001) (end 122.083999 44.097001) (width 0.25) (layer F.Cu) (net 5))
 (segment (start 122.018999 33.937001) (end 122.018999 44.032001) (width 0.25) (layer F.Cu) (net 5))
 (segment (start 123.444 32.512) (end 122.018999 33.937001) (width 0.25) (layer F.Cu) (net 5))
 (segment (start 129.519827 44.049) (end 129.519827 46.409) (width 0.25) (layer F.Cu) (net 5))
 (segment (start 100.584 43.371) (end 102.616 45.403) (width 0.25) (layer F.Cu) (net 7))
 (segment (start 100.584 39.116) (end 100.584 43.371) (width 0.25) (layer F.Cu) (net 7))
 (segment (start 129.519827 42.399) (end 129.519827 40.039) (width 0.25) (layer F.Cu) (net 9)))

